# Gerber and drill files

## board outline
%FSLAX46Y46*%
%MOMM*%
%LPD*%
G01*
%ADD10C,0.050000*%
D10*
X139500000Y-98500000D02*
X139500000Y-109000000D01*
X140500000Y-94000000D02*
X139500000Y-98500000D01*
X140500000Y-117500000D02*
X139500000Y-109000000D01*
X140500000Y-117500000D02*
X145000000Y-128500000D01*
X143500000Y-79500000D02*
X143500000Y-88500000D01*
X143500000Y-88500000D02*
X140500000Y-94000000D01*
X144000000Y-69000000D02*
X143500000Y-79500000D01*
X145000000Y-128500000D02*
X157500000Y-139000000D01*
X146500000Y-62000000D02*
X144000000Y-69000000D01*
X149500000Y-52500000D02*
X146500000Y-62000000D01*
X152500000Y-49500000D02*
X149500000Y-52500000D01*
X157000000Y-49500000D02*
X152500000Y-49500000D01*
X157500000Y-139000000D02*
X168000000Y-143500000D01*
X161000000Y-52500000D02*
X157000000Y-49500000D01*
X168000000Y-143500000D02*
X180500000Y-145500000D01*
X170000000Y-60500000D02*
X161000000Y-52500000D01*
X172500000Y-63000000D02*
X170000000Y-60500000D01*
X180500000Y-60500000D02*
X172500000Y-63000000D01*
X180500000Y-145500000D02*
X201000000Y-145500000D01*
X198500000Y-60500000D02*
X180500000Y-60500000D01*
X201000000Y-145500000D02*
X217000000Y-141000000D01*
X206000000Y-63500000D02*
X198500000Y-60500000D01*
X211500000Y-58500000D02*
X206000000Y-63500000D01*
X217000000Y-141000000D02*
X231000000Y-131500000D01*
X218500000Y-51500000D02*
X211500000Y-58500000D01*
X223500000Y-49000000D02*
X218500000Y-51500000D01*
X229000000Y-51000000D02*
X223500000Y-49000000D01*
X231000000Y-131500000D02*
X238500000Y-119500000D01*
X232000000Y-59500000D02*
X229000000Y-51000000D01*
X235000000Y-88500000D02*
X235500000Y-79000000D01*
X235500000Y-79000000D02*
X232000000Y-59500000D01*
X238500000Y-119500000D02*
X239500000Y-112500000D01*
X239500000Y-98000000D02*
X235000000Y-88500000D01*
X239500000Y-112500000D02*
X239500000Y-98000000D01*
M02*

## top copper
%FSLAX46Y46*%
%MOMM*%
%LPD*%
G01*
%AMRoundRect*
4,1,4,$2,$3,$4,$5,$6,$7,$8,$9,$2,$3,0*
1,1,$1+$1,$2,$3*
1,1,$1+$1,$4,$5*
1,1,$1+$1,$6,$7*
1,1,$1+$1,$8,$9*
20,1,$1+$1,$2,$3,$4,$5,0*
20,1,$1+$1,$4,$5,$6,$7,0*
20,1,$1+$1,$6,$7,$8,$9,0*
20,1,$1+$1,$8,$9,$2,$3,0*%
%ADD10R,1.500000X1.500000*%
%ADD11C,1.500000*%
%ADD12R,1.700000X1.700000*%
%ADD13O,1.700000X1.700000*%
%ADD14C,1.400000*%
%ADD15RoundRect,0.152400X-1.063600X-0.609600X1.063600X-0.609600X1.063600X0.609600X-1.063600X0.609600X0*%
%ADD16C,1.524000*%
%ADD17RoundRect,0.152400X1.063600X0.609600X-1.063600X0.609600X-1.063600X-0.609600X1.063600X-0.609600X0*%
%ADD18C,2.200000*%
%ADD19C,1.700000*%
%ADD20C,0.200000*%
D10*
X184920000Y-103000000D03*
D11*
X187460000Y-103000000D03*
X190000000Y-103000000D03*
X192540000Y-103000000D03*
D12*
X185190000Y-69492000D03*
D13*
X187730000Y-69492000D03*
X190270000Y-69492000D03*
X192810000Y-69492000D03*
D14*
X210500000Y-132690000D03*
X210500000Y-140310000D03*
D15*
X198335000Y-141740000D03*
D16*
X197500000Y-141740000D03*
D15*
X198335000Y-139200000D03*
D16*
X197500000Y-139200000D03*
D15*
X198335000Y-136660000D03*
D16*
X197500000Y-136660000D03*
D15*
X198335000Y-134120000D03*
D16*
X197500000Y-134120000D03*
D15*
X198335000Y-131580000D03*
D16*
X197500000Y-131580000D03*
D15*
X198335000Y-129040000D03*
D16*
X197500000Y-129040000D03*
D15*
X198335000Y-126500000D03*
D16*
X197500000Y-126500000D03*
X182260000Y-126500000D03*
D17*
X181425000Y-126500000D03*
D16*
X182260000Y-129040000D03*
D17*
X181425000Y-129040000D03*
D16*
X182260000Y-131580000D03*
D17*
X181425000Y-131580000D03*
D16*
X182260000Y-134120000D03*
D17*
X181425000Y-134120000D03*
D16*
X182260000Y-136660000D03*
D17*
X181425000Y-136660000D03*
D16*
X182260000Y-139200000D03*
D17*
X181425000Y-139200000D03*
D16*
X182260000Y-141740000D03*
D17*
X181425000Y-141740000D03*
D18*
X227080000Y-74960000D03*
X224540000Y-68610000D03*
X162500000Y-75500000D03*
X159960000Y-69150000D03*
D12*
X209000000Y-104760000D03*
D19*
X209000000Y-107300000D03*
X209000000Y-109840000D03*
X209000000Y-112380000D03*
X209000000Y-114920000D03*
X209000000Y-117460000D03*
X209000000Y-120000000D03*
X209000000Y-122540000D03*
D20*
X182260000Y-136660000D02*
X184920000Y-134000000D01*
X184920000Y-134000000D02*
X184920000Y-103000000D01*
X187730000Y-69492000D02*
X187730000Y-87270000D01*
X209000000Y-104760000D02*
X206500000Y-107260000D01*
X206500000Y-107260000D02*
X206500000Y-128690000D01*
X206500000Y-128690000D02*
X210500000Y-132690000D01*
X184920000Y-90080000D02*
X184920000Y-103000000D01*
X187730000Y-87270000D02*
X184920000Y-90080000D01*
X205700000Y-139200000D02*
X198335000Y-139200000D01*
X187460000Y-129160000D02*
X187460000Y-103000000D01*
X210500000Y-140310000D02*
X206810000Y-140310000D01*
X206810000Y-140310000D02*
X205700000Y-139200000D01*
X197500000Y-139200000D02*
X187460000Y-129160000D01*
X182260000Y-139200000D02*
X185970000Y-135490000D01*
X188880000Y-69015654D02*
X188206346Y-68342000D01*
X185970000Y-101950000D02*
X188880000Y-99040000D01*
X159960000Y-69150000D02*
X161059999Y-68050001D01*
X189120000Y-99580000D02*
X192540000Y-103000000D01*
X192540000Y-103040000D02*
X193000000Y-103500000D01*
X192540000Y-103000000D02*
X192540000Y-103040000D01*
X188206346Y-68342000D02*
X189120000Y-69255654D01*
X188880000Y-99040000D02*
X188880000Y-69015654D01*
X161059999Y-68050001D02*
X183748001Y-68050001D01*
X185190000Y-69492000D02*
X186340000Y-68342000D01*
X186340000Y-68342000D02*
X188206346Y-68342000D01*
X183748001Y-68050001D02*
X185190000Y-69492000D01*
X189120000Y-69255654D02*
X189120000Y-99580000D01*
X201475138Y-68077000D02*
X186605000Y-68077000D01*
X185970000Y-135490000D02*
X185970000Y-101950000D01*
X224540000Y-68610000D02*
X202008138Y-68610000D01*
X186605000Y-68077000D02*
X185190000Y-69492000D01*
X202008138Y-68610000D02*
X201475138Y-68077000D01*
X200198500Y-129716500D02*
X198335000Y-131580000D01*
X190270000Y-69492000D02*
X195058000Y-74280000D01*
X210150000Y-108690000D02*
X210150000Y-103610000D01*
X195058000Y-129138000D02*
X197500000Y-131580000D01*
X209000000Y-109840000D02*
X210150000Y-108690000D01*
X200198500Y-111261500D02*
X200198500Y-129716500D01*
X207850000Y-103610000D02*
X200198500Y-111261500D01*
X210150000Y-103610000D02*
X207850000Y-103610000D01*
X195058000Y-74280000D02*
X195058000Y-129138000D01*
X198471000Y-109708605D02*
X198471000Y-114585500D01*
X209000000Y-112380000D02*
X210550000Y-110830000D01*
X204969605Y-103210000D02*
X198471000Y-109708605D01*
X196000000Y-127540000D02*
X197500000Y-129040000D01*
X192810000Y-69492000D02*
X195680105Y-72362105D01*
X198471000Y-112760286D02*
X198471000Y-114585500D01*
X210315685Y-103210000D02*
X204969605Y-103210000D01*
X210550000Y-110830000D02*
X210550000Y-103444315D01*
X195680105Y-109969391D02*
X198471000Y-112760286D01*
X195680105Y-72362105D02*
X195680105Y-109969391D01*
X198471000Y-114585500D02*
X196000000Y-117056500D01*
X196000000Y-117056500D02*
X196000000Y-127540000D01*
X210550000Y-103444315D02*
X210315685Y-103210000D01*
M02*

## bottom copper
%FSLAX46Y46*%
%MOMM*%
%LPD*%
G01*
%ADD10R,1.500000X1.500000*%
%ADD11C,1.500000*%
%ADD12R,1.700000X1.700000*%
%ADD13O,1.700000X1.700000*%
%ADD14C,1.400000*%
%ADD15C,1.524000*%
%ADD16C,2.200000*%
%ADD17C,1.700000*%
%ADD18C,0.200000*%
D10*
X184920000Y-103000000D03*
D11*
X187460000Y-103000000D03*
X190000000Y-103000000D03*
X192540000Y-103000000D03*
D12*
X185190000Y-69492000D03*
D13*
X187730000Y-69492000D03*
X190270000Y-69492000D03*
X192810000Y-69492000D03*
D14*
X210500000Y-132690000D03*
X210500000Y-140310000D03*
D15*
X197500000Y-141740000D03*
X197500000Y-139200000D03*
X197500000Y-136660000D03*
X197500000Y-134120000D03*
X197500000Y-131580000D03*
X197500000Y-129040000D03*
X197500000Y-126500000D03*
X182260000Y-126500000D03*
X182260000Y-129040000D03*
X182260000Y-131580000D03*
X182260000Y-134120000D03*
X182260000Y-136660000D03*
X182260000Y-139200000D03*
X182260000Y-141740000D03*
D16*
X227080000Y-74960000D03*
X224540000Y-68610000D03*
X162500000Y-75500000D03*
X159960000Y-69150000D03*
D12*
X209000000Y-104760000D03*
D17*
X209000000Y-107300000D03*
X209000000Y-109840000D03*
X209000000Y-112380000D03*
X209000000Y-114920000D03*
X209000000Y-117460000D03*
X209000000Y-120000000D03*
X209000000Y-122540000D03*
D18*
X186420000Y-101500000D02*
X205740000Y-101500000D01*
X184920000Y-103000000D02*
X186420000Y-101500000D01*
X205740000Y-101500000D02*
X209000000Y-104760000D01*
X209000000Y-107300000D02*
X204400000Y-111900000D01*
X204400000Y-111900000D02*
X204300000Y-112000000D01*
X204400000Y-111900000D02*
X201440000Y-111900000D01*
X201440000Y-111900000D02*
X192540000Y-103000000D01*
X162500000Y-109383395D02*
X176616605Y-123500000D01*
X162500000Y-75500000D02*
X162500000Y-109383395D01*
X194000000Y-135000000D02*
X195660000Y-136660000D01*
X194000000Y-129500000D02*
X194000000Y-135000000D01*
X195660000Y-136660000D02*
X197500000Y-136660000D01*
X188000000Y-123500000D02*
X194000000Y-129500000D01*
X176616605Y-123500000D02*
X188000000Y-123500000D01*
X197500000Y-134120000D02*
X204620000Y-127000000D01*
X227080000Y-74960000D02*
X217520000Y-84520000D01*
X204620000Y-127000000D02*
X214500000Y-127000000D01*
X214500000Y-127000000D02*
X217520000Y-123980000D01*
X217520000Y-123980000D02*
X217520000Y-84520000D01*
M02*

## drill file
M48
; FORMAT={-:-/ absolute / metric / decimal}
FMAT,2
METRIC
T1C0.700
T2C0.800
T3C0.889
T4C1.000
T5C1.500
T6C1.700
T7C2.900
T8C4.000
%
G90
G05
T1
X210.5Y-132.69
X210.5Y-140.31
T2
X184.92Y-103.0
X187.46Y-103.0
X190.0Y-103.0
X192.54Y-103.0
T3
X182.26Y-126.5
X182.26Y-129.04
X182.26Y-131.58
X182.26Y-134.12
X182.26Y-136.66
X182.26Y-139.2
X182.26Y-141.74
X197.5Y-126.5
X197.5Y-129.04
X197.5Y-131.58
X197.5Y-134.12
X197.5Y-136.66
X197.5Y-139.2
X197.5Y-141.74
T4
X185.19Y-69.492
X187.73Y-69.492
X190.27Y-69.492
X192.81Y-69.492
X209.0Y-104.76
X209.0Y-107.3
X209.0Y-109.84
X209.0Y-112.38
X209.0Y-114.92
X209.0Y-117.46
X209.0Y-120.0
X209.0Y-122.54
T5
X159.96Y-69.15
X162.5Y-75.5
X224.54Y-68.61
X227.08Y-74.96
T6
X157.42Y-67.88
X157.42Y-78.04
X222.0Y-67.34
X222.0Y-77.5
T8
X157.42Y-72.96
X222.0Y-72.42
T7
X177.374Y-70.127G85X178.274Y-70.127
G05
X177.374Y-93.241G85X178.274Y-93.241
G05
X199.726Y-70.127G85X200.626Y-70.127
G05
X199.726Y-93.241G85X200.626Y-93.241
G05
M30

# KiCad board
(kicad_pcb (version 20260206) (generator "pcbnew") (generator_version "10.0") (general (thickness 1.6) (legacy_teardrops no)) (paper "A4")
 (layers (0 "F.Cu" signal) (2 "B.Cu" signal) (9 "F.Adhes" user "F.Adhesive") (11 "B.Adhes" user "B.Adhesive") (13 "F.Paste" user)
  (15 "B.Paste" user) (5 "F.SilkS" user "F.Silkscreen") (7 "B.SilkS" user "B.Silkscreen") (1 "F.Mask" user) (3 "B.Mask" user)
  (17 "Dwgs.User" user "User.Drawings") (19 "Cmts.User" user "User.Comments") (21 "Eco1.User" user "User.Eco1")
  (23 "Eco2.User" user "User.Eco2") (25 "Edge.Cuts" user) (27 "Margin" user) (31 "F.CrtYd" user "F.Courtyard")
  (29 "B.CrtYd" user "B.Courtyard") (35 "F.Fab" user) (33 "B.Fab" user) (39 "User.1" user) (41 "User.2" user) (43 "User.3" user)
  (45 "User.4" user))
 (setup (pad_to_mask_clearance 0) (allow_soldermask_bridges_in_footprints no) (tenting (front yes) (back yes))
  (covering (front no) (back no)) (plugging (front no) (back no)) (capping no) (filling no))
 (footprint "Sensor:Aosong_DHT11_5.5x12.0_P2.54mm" (layer "F.Cu") (at 184.92 103 90)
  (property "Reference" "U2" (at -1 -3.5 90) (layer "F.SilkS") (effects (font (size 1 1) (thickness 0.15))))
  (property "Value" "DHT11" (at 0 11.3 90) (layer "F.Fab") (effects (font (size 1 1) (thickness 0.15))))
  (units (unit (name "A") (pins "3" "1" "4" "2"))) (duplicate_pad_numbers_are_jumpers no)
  (pad "1" thru_hole rect (at 0 0 90) (size 1.5 1.5) (drill 0.8) (layers "*.Cu" "*.Mask") (remove_unused_layers no) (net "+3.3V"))
  (pad "2" thru_hole circle (at 0 2.54 90) (size 1.5 1.5) (drill 0.8) (layers "*.Cu" "*.Mask") (remove_unused_layers no) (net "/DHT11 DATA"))
  (pad "3" thru_hole circle (at 0 5.08 90) (size 1.5 1.5) (drill 0.8) (layers "*.Cu" "*.Mask") (remove_unused_layers no)
   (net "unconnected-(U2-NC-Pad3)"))
  (pad "4" thru_hole circle (at 0 7.62 90) (size 1.5 1.5) (drill 0.8) (layers "*.Cu" "*.Mask") (remove_unused_layers no) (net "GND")))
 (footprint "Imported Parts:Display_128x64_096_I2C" (layer "F.Cu") (at 189 69.492)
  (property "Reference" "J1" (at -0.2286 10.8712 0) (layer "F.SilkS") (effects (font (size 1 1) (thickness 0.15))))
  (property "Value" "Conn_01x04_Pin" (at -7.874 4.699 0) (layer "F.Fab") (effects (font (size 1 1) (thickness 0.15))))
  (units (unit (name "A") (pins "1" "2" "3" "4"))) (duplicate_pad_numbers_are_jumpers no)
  (pad "" np_thru_hole oval (at -11.176 0.635) (size 3.8 2.9) (drill oval 3.8 2.9) (layers "*.Cu" "*.Mask"))
  (pad "" np_thru_hole oval (at -11.176 23.749) (size 3.8 2.9) (drill oval 3.8 2.9) (layers "*.Cu" "*.Mask"))
  (pad "" np_thru_hole oval (at 11.176 0.635) (size 3.8 2.9) (drill oval 3.8 2.9) (layers "*.Cu" "*.Mask"))
  (pad "" np_thru_hole oval (at 11.176 23.749) (size 3.8 2.9) (drill oval 3.8 2.9) (layers "*.Cu" "*.Mask"))
  (pad "1" thru_hole rect (at -3.81 0 90) (size 1.7 1.7) (drill 1) (layers "*.Cu" "*.Mask") (remove_unused_layers no) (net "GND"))
  (pad "2" thru_hole oval (at -1.27 0 90) (size 1.7 1.7) (drill 1) (layers "*.Cu" "*.Mask") (remove_unused_layers no) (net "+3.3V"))
  (pad "3" thru_hole oval (at 1.27 0 90) (size 1.7 1.7) (drill 1) (layers "*.Cu" "*.Mask") (remove_unused_layers no) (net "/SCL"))
  (pad "4" thru_hole oval (at 3.81 0 90) (size 1.7 1.7) (drill 1) (layers "*.Cu" "*.Mask") (remove_unused_layers no) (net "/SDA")))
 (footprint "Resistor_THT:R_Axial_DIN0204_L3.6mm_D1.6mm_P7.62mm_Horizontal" (layer "F.Cu") (at 210.5 132.69 -90)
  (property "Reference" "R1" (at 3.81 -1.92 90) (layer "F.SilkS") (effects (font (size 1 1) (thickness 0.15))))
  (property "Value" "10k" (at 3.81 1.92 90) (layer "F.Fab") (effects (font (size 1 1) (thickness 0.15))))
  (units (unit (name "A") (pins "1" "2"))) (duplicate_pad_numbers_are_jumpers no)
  (pad "1" thru_hole circle (at 0 0 270) (size 1.4 1.4) (drill 0.7) (layers "*.Cu" "*.Mask") (remove_unused_layers no) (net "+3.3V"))
  (pad "2" thru_hole circle (at 7.62 0 270) (size 1.4 1.4) (drill 0.7) (layers "*.Cu" "*.Mask") (remove_unused_layers no)
   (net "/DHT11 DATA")))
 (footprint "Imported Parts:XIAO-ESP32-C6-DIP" (layer "F.Cu") (at 189.88 134.12 -90)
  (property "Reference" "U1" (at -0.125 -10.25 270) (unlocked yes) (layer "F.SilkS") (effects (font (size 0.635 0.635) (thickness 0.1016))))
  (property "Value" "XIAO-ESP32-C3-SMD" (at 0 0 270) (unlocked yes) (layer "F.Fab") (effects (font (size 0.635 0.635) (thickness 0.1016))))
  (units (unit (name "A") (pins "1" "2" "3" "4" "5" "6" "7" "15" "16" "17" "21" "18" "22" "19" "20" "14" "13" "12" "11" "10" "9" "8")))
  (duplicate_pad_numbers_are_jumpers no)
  (pad "1" smd roundrect (at 7.62 -8.455) (size 2.432 1.524) (layers "F.Cu" "F.Mask") (roundrect_rratio 0.1)
   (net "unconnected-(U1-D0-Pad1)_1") (thermal_bridge_angle 45))
  (pad "1" thru_hole circle (at 7.62 -7.62) (size 1.524 1.524) (drill 0.889) (layers "*.Cu" "*.Mask") (remove_unused_layers no)
   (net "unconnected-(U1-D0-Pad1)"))
  (pad "2" smd roundrect (at 5.08 -8.455) (size 2.432 1.524) (layers "F.Cu" "F.Mask") (roundrect_rratio 0.1) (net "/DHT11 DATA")
   (thermal_bridge_angle 45))
  (pad "2" thru_hole circle (at 5.08 -7.62) (size 1.524 1.524) (drill 0.889) (layers "*.Cu" "*.Mask") (remove_unused_layers no)
   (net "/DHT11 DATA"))
  (pad "3" smd roundrect (at 2.54 -8.455) (size 2.432 1.524) (layers "F.Cu" "F.Mask") (roundrect_rratio 0.1) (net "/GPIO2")
   (thermal_bridge_angle 45))
  (pad "3" thru_hole circle (at 2.54 -7.62) (size 1.524 1.524) (drill 0.889) (layers "*.Cu" "*.Mask") (remove_unused_layers no)
   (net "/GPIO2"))
  (pad "4" smd roundrect (at 0 -8.455) (size 2.432 1.524) (layers "F.Cu" "F.Mask") (roundrect_rratio 0.1) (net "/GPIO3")
   (thermal_bridge_angle 45))
  (pad "4" thru_hole circle (at 0 -7.62) (size 1.524 1.524) (drill 0.889) (layers "*.Cu" "*.Mask") (remove_unused_layers no) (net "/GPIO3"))
  (pad "5" smd roundrect (at -2.54 -8.455) (size 2.432 1.524) (layers "F.Cu" "F.Mask") (roundrect_rratio 0.1) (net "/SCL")
   (thermal_bridge_angle 45))
  (pad "5" thru_hole circle (at -2.54 -7.62) (size 1.524 1.524) (drill 0.889) (layers "*.Cu" "*.Mask") (remove_unused_layers no)
   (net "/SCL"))
  (pad "6" smd roundrect (at -5.08 -8.455) (size 2.432 1.524) (layers "F.Cu" "F.Mask") (roundrect_rratio 0.1) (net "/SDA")
   (thermal_bridge_angle 45))
  (pad "6" thru_hole circle (at -5.08 -7.62) (size 1.524 1.524) (drill 0.889) (layers "*.Cu" "*.Mask") (remove_unused_layers no)
   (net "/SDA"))
  (pad "7" smd roundrect (at -7.62 -8.455) (size 2.432 1.524) (layers "F.Cu" "F.Mask") (roundrect_rratio 0.1)
   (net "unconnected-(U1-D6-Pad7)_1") (thermal_bridge_angle 45))
  (pad "7" thru_hole circle (at -7.62 -7.62) (size 1.524 1.524) (drill 0.889) (layers "*.Cu" "*.Mask") (remove_unused_layers no)
   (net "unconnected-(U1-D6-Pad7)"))
  (pad "8" thru_hole circle (at -7.62 7.62 180) (size 1.524 1.524) (drill 0.889) (layers "*.Cu" "*.Mask") (remove_unused_layers no)
   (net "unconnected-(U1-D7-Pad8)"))
  (pad "8" smd roundrect (at -7.62 8.455 180) (size 2.432 1.524) (layers "F.Cu" "F.Mask") (roundrect_rratio 0.1)
   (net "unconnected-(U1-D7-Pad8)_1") (thermal_bridge_angle 45))
  (pad "9" thru_hole circle (at -5.08 7.62 180) (size 1.524 1.524) (drill 0.889) (layers "*.Cu" "*.Mask") (remove_unused_layers no)
   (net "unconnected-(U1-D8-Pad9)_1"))
  (pad "9" smd roundrect (at -5.08 8.455 180) (size 2.432 1.524) (layers "F.Cu" "F.Mask") (roundrect_rratio 0.1)
   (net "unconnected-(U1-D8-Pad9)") (thermal_bridge_angle 45))
  (pad "10" thru_hole circle (at -2.54 7.62 180) (size 1.524 1.524) (drill 0.889) (layers "*.Cu" "*.Mask") (remove_unused_layers no)
   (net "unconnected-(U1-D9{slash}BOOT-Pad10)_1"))
  (pad "10" smd roundrect (at -2.54 8.455 180) (size 2.432 1.524) (layers "F.Cu" "F.Mask") (roundrect_rratio 0.1)
   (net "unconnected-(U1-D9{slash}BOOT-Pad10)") (thermal_bridge_angle 45))
  (pad "11" thru_hole circle (at 0 7.62 180) (size 1.524 1.524) (drill 0.889) (layers "*.Cu" "*.Mask") (remove_unused_layers no)
   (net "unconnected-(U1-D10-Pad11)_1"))
  (pad "11" smd roundrect (at 0 8.455 180) (size 2.432 1.524) (layers "F.Cu" "F.Mask") (roundrect_rratio 0.1)
   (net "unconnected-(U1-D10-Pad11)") (thermal_bridge_angle 45))
  (pad "12" thru_hole circle (at 2.54 7.62 180) (size 1.524 1.524) (drill 0.889) (layers "*.Cu" "*.Mask") (remove_unused_layers no)
   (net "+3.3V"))
  (pad "12" smd roundrect (at 2.54 8.455 180) (size 2.432 1.524) (layers "F.Cu" "F.Mask") (roundrect_rratio 0.1) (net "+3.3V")
   (thermal_bridge_angle 45))
  (pad "13" thru_hole circle (at 5.08 7.62 180) (size 1.524 1.524) (drill 0.889) (layers "*.Cu" "*.Mask") (remove_unused_layers no)
   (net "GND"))
  (pad "13" smd roundrect (at 5.08 8.455 180) (size 2.432 1.524) (layers "F.Cu" "F.Mask") (roundrect_rratio 0.1) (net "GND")
   (thermal_bridge_angle 45))
  (pad "14" thru_hole circle (at 7.62 7.62 180) (size 1.524 1.524) (drill 0.889) (layers "*.Cu" "*.Mask") (remove_unused_layers no)
   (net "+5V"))
  (pad "14" smd roundrect (at 7.62 8.455 180) (size 2.432 1.524) (layers "F.Cu" "F.Mask") (roundrect_rratio 0.1) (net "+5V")
   (thermal_bridge_angle 45)))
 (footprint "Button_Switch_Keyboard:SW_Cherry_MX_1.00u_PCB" (layer "F.Cu") (at 227.08 74.96 -90)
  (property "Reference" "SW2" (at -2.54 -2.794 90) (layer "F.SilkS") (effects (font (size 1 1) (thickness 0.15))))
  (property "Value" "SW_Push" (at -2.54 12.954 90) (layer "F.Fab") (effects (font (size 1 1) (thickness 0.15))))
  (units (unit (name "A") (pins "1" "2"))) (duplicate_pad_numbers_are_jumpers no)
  (pad "" np_thru_hole circle (at -7.62 5.08 270) (size 1.7 1.7) (drill 1.7) (layers "*.Cu" "*.Mask"))
  (pad "" np_thru_hole circle (at -2.54 5.08 270) (size 4 4) (drill 4) (layers "*.Cu" "*.Mask"))
  (pad "" np_thru_hole circle (at 2.54 5.08 270) (size 1.7 1.7) (drill 1.7) (layers "*.Cu" "*.Mask"))
  (pad "1" thru_hole circle (at 0 0 270) (size 2.2 2.2) (drill 1.5) (layers "*.Cu" "*.Mask") (remove_unused_layers no) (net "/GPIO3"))
  (pad "2" thru_hole circle (at -6.35 2.54 270) (size 2.2 2.2) (drill 1.5) (layers "*.Cu" "*.Mask") (remove_unused_layers no) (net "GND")))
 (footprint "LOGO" (layer "F.Cu") (at 160.5 102)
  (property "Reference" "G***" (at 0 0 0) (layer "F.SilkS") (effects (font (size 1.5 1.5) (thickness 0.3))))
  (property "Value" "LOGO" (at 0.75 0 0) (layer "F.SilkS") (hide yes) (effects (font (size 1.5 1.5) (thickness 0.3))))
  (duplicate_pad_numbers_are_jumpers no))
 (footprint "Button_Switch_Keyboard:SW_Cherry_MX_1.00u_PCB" (layer "F.Cu") (at 162.5 75.5 -90)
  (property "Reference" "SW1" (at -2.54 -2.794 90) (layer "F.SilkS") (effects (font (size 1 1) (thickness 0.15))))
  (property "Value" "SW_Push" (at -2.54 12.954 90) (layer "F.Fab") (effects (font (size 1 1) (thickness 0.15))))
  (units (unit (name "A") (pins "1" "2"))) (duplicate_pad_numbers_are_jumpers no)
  (pad "" np_thru_hole circle (at -7.62 5.08 270) (size 1.7 1.7) (drill 1.7) (layers "*.Cu" "*.Mask"))
  (pad "" np_thru_hole circle (at -2.54 5.08 270) (size 4 4) (drill 4) (layers "*.Cu" "*.Mask"))
  (pad "" np_thru_hole circle (at 2.54 5.08 270) (size 1.7 1.7) (drill 1.7) (layers "*.Cu" "*.Mask"))
  (pad "1" thru_hole circle (at 0 0 270) (size 2.2 2.2) (drill 1.5) (layers "*.Cu" "*.Mask") (remove_unused_layers no) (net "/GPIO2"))
  (pad "2" thru_hole circle (at -6.35 2.54 270) (size 2.2 2.2) (drill 1.5) (layers "*.Cu" "*.Mask") (remove_unused_layers no) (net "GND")))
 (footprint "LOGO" (layer "F.Cu") (at 221.320709 88.876762)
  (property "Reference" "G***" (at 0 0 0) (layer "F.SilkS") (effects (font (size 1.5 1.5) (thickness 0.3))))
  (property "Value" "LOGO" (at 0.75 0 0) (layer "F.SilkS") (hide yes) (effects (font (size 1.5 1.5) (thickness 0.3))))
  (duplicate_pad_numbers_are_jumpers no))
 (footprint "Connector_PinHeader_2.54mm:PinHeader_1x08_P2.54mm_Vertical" (layer "F.Cu") (at 209 104.76)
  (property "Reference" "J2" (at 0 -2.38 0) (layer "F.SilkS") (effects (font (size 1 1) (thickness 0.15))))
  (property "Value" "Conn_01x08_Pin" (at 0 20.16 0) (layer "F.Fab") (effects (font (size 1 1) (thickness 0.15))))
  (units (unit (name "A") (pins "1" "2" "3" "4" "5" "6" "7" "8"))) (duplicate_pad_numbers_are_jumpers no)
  (pad "1" thru_hole rect (at 0 0) (size 1.7 1.7) (drill 1) (layers "*.Cu" "*.Mask") (remove_unused_layers no) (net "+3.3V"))
  (pad "2" thru_hole circle (at 0 2.54) (size 1.7 1.7) (drill 1) (layers "*.Cu" "*.Mask") (remove_unused_layers no) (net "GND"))
  (pad "3" thru_hole circle (at 0 5.08) (size 1.7 1.7) (drill 1) (layers "*.Cu" "*.Mask") (remove_unused_layers no) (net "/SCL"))
  (pad "4" thru_hole circle (at 0 7.62) (size 1.7 1.7) (drill 1) (layers "*.Cu" "*.Mask") (remove_unused_layers no) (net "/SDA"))
  (pad "5" thru_hole circle (at 0 10.16) (size 1.7 1.7) (drill 1) (layers "*.Cu" "*.Mask") (remove_unused_layers no)
   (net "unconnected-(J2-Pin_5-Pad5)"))
  (pad "6" thru_hole circle (at 0 12.7) (size 1.7 1.7) (drill 1) (layers "*.Cu" "*.Mask") (remove_unused_layers no)
   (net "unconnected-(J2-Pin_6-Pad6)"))
  (pad "7" thru_hole circle (at 0 15.24) (size 1.7 1.7) (drill 1) (layers "*.Cu" "*.Mask") (remove_unused_layers no)
   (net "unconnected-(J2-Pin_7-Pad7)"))
  (pad "8" thru_hole circle (at 0 17.78) (size 1.7 1.7) (drill 1) (layers "*.Cu" "*.Mask") (remove_unused_layers no)
   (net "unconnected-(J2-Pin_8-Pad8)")))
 (gr_line (start 139.5 98.5) (end 139.5 109) (stroke (width 0.05) (type default)) (layer "Edge.Cuts"))
 (gr_line (start 140.5 94) (end 139.5 98.5) (stroke (width 0.05) (type default)) (layer "Edge.Cuts"))
 (gr_line (start 140.5 117.5) (end 139.5 109) (stroke (width 0.05) (type default)) (layer "Edge.Cuts"))
 (gr_line (start 140.5 117.5) (end 145 128.5) (stroke (width 0.05) (type default)) (layer "Edge.Cuts"))
 (gr_line (start 143.5 79.5) (end 143.5 88.5) (stroke (width 0.05) (type default)) (layer "Edge.Cuts"))
 (gr_line (start 143.5 88.5) (end 140.5 94) (stroke (width 0.05) (type default)) (layer "Edge.Cuts"))
 (gr_line (start 144 69) (end 143.5 79.5) (stroke (width 0.05) (type default)) (layer "Edge.Cuts"))
 (gr_line (start 145 128.5) (end 157.5 139) (stroke (width 0.05) (type default)) (layer "Edge.Cuts"))
 (gr_line (start 146.5 62) (end 144 69) (stroke (width 0.05) (type default)) (layer "Edge.Cuts"))
 (gr_line (start 149.5 52.5) (end 146.5 62) (stroke (width 0.05) (type default)) (layer "Edge.Cuts"))
 (gr_line (start 152.5 49.5) (end 149.5 52.5) (stroke (width 0.05) (type default)) (layer "Edge.Cuts"))
 (gr_line (start 157 49.5) (end 152.5 49.5) (stroke (width 0.05) (type default)) (layer "Edge.Cuts"))
 (gr_line (start 157.5 139) (end 168 143.5) (stroke (width 0.05) (type default)) (layer "Edge.Cuts"))
 (gr_line (start 161 52.5) (end 157 49.5) (stroke (width 0.05) (type default)) (layer "Edge.Cuts"))
 (gr_line (start 168 143.5) (end 180.5 145.5) (stroke (width 0.05) (type default)) (layer "Edge.Cuts"))
 (gr_line (start 170 60.5) (end 161 52.5) (stroke (width 0.05) (type default)) (layer "Edge.Cuts"))
 (gr_line (start 172.5 63) (end 170 60.5) (stroke (width 0.05) (type default)) (layer "Edge.Cuts"))
 (gr_line (start 180.5 60.5) (end 172.5 63) (stroke (width 0.05) (type default)) (layer "Edge.Cuts"))
 (gr_line (start 180.5 145.5) (end 201 145.5) (stroke (width 0.05) (type default)) (layer "Edge.Cuts"))
 (gr_line (start 198.5 60.5) (end 180.5 60.5) (stroke (width 0.05) (type default)) (layer "Edge.Cuts"))
 (gr_line (start 201 145.5) (end 217 141) (stroke (width 0.05) (type default)) (layer "Edge.Cuts"))
 (gr_line (start 206 63.5) (end 198.5 60.5) (stroke (width 0.05) (type default)) (layer "Edge.Cuts"))
 (gr_line (start 211.5 58.5) (end 206 63.5) (stroke (width 0.05) (type default)) (layer "Edge.Cuts"))
 (gr_line (start 217 141) (end 231 131.5) (stroke (width 0.05) (type default)) (layer "Edge.Cuts"))
 (gr_line (start 218.5 51.5) (end 211.5 58.5) (stroke (width 0.05) (type default)) (layer "Edge.Cuts"))
 (gr_line (start 223.5 49) (end 218.5 51.5) (stroke (width 0.05) (type default)) (layer "Edge.Cuts"))
 (gr_line (start 229 51) (end 223.5 49) (stroke (width 0.05) (type default)) (layer "Edge.Cuts"))
 (gr_line (start 231 131.5) (end 238.5 119.5) (stroke (width 0.05) (type default)) (layer "Edge.Cuts"))
 (gr_line (start 232 59.5) (end 229 51) (stroke (width 0.05) (type default)) (layer "Edge.Cuts"))
 (gr_line (start 235 88.5) (end 235.5 79) (stroke (width 0.05) (type default)) (layer "Edge.Cuts"))
 (gr_line (start 235.5 79) (end 232 59.5) (stroke (width 0.05) (type default)) (layer "Edge.Cuts"))
 (gr_line (start 238.5 119.5) (end 239.5 112.5) (stroke (width 0.05) (type default)) (layer "Edge.Cuts"))
 (gr_line (start 239.5 98) (end 235 88.5) (stroke (width 0.05) (type default)) (layer "Edge.Cuts"))
 (gr_line (start 239.5 112.5) (end 239.5 98) (stroke (width 0.05) (type default)) (layer "Edge.Cuts"))
 (segment (start 182.26 136.66) (end 184.92 134) (width 0.2) (layer "F.Cu") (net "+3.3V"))
 (segment (start 184.92 134) (end 184.92 103) (width 0.2) (layer "F.Cu") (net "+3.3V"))
 (segment (start 187.73 69.492) (end 187.73 87.27) (width 0.2) (layer "F.Cu") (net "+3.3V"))
 (segment (start 209 104.76) (end 206.5 107.26) (width 0.2) (layer "F.Cu") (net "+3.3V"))
 (segment (start 206.5 107.26) (end 206.5 128.69) (width 0.2) (layer "F.Cu") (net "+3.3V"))
 (segment (start 206.5 128.69) (end 210.5 132.69) (width 0.2) (layer "F.Cu") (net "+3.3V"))
 (segment (start 184.92 90.08) (end 184.92 103) (width 0.2) (layer "F.Cu") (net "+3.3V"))
 (segment (start 187.73 87.27) (end 184.92 90.08) (width 0.2) (layer "F.Cu") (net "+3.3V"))
 (segment (start 186.42 101.5) (end 205.74 101.5) (width 0.2) (layer "B.Cu") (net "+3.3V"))
 (segment (start 184.92 103) (end 186.42 101.5) (width 0.2) (layer "B.Cu") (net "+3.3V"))
 (segment (start 205.74 101.5) (end 209 104.76) (width 0.2) (layer "B.Cu") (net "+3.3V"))
 (segment (start 205.7 139.2) (end 198.335 139.2) (width 0.2) (layer "F.Cu") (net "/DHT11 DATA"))
 (segment (start 187.46 129.16) (end 187.46 103) (width 0.2) (layer "F.Cu") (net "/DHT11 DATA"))
 (segment (start 210.5 140.31) (end 206.81 140.31) (width 0.2) (layer "F.Cu") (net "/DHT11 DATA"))
 (segment (start 206.81 140.31) (end 205.7 139.2) (width 0.2) (layer "F.Cu") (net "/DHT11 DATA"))
 (segment (start 197.5 139.2) (end 187.46 129.16) (width 0.2) (layer "F.Cu") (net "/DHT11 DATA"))
 (segment (start 182.26 139.2) (end 185.97 135.49) (width 0.2) (layer "F.Cu") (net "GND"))
 (segment (start 188.88 69.015654) (end 188.206346 68.342) (width 0.2) (layer "F.Cu") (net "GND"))
 (segment (start 185.97 101.95) (end 188.88 99.04) (width 0.2) (layer "F.Cu") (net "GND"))
 (segment (start 159.96 69.15) (end 161.059999 68.050001) (width 0.2) (layer "F.Cu") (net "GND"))
 (segment (start 189.12 99.58) (end 192.54 103) (width 0.2) (layer "F.Cu") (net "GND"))
 (segment (start 192.54 103.04) (end 193 103.5) (width 0.2) (layer "F.Cu") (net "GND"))
 (segment (start 192.54 103) (end 192.54 103.04) (width 0.2) (layer "F.Cu") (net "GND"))
 (segment (start 188.206346 68.342) (end 189.12 69.255654) (width 0.2) (layer "F.Cu") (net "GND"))
 (segment (start 188.88 99.04) (end 188.88 69.015654) (width 0.2) (layer "F.Cu") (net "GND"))
 (segment (start 161.059999 68.050001) (end 183.748001 68.050001) (width 0.2) (layer "F.Cu") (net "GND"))
 (segment (start 185.19 69.492) (end 186.34 68.342) (width 0.2) (layer "F.Cu") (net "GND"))
 (segment (start 186.34 68.342) (end 188.206346 68.342) (width 0.2) (layer "F.Cu") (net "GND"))
 (segment (start 183.748001 68.050001) (end 185.19 69.492) (width 0.2) (layer "F.Cu") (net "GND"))
 (segment (start 189.12 69.255654) (end 189.12 99.58) (width 0.2) (layer "F.Cu") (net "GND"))
 (segment (start 201.475138 68.077) (end 186.605 68.077) (width 0.2) (layer "F.Cu") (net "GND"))
 (segment (start 185.97 135.49) (end 185.97 101.95) (width 0.2) (layer "F.Cu") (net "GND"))
 (segment (start 224.54 68.61) (end 202.008138 68.61) (width 0.2) (layer "F.Cu") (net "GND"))
 (segment (start 186.605 68.077) (end 185.19 69.492) (width 0.2) (layer "F.Cu") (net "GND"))
 (segment (start 202.008138 68.61) (end 201.475138 68.077) (width 0.2) (layer "F.Cu") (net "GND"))
 (segment (start 209 107.3) (end 204.4 111.9) (width 0.2) (layer "B.Cu") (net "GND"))
 (segment (start 204.4 111.9) (end 204.3 112) (width 0.2) (layer "B.Cu") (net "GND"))
 (segment (start 204.4 111.9) (end 201.44 111.9) (width 0.2) (layer "B.Cu") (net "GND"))
 (segment (start 201.44 111.9) (end 192.54 103) (width 0.2) (layer "B.Cu") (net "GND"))
 (segment (start 200.1985 129.7165) (end 198.335 131.58) (width 0.2) (layer "F.Cu") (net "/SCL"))
 (segment (start 190.27 69.492) (end 195.058 74.28) (width 0.2) (layer "F.Cu") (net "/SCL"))
 (segment (start 210.15 108.69) (end 210.15 103.61) (width 0.2) (layer "F.Cu") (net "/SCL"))
 (segment (start 195.058 129.138) (end 197.5 131.58) (width 0.2) (layer "F.Cu") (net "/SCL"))
 (segment (start 209 109.84) (end 210.15 108.69) (width 0.2) (layer "F.Cu") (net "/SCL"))
 (segment (start 200.1985 111.2615) (end 200.1985 129.7165) (width 0.2) (layer "F.Cu") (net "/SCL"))
 (segment (start 207.85 103.61) (end 200.1985 111.2615) (width 0.2) (layer "F.Cu") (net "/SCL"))
 (segment (start 210.15 103.61) (end 207.85 103.61) (width 0.2) (layer "F.Cu") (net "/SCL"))
 (segment (start 195.058 74.28) (end 195.058 129.138) (width 0.2) (layer "F.Cu") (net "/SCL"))
 (segment (start 198.471 109.708605) (end 198.471 114.5855) (width 0.2) (layer "F.Cu") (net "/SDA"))
 (segment (start 209 112.38) (end 210.55 110.83) (width 0.2) (layer "F.Cu") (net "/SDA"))
 (segment (start 204.969605 103.21) (end 198.471 109.708605) (width 0.2) (layer "F.Cu") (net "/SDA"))
 (segment (start 196 127.54) (end 197.5 129.04) (width 0.2) (layer "F.Cu") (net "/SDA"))
 (segment (start 192.81 69.492) (end 195.680105 72.362105) (width 0.2) (layer "F.Cu") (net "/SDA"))
 (segment (start 198.471 112.760286) (end 198.471 114.5855) (width 0.2) (layer "F.Cu") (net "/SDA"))
 (segment (start 210.315685 103.21) (end 204.969605 103.21) (width 0.2) (layer "F.Cu") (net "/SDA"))
 (segment (start 210.55 110.83) (end 210.55 103.444315) (width 0.2) (layer "F.Cu") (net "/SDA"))
 (segment (start 195.680105 109.969391) (end 198.471 112.760286) (width 0.2) (layer "F.Cu") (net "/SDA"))
 (segment (start 195.680105 72.362105) (end 195.680105 109.969391) (width 0.2) (layer "F.Cu") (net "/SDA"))
 (segment (start 198.471 114.5855) (end 196 117.0565) (width 0.2) (layer "F.Cu") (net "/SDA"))
 (segment (start 196 117.0565) (end 196 127.54) (width 0.2) (layer "F.Cu") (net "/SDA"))
 (segment (start 210.55 103.444315) (end 210.315685 103.21) (width 0.2) (layer "F.Cu") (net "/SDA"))
 (segment (start 162.5 109.383395) (end 176.616605 123.5) (width 0.2) (layer "B.Cu") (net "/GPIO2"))
 (segment (start 162.5 75.5) (end 162.5 109.383395) (width 0.2) (layer "B.Cu") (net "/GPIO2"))
 (segment (start 194 135) (end 195.66 136.66) (width 0.2) (layer "B.Cu") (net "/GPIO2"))
 (segment (start 194 129.5) (end 194 135) (width 0.2) (layer "B.Cu") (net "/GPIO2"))
 (segment (start 195.66 136.66) (end 197.5 136.66) (width 0.2) (layer "B.Cu") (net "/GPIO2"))
 (segment (start 188 123.5) (end 194 129.5) (width 0.2) (layer "B.Cu") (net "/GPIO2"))
 (segment (start 176.616605 123.5) (end 188 123.5) (width 0.2) (layer "B.Cu") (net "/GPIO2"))
 (segment (start 197.5 134.12) (end 204.62 127) (width 0.2) (layer "B.Cu") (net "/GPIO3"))
 (segment (start 227.08 74.96) (end 217.52 84.52) (width 0.2) (layer "B.Cu") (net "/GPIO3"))
 (segment (start 204.62 127) (end 214.5 127) (width 0.2) (layer "B.Cu") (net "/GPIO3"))
 (segment (start 214.5 127) (end 217.52 123.98) (width 0.2) (layer "B.Cu") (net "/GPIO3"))
 (segment (start 217.52 123.98) (end 217.52 84.52) (width 0.2) (layer "B.Cu") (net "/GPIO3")))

